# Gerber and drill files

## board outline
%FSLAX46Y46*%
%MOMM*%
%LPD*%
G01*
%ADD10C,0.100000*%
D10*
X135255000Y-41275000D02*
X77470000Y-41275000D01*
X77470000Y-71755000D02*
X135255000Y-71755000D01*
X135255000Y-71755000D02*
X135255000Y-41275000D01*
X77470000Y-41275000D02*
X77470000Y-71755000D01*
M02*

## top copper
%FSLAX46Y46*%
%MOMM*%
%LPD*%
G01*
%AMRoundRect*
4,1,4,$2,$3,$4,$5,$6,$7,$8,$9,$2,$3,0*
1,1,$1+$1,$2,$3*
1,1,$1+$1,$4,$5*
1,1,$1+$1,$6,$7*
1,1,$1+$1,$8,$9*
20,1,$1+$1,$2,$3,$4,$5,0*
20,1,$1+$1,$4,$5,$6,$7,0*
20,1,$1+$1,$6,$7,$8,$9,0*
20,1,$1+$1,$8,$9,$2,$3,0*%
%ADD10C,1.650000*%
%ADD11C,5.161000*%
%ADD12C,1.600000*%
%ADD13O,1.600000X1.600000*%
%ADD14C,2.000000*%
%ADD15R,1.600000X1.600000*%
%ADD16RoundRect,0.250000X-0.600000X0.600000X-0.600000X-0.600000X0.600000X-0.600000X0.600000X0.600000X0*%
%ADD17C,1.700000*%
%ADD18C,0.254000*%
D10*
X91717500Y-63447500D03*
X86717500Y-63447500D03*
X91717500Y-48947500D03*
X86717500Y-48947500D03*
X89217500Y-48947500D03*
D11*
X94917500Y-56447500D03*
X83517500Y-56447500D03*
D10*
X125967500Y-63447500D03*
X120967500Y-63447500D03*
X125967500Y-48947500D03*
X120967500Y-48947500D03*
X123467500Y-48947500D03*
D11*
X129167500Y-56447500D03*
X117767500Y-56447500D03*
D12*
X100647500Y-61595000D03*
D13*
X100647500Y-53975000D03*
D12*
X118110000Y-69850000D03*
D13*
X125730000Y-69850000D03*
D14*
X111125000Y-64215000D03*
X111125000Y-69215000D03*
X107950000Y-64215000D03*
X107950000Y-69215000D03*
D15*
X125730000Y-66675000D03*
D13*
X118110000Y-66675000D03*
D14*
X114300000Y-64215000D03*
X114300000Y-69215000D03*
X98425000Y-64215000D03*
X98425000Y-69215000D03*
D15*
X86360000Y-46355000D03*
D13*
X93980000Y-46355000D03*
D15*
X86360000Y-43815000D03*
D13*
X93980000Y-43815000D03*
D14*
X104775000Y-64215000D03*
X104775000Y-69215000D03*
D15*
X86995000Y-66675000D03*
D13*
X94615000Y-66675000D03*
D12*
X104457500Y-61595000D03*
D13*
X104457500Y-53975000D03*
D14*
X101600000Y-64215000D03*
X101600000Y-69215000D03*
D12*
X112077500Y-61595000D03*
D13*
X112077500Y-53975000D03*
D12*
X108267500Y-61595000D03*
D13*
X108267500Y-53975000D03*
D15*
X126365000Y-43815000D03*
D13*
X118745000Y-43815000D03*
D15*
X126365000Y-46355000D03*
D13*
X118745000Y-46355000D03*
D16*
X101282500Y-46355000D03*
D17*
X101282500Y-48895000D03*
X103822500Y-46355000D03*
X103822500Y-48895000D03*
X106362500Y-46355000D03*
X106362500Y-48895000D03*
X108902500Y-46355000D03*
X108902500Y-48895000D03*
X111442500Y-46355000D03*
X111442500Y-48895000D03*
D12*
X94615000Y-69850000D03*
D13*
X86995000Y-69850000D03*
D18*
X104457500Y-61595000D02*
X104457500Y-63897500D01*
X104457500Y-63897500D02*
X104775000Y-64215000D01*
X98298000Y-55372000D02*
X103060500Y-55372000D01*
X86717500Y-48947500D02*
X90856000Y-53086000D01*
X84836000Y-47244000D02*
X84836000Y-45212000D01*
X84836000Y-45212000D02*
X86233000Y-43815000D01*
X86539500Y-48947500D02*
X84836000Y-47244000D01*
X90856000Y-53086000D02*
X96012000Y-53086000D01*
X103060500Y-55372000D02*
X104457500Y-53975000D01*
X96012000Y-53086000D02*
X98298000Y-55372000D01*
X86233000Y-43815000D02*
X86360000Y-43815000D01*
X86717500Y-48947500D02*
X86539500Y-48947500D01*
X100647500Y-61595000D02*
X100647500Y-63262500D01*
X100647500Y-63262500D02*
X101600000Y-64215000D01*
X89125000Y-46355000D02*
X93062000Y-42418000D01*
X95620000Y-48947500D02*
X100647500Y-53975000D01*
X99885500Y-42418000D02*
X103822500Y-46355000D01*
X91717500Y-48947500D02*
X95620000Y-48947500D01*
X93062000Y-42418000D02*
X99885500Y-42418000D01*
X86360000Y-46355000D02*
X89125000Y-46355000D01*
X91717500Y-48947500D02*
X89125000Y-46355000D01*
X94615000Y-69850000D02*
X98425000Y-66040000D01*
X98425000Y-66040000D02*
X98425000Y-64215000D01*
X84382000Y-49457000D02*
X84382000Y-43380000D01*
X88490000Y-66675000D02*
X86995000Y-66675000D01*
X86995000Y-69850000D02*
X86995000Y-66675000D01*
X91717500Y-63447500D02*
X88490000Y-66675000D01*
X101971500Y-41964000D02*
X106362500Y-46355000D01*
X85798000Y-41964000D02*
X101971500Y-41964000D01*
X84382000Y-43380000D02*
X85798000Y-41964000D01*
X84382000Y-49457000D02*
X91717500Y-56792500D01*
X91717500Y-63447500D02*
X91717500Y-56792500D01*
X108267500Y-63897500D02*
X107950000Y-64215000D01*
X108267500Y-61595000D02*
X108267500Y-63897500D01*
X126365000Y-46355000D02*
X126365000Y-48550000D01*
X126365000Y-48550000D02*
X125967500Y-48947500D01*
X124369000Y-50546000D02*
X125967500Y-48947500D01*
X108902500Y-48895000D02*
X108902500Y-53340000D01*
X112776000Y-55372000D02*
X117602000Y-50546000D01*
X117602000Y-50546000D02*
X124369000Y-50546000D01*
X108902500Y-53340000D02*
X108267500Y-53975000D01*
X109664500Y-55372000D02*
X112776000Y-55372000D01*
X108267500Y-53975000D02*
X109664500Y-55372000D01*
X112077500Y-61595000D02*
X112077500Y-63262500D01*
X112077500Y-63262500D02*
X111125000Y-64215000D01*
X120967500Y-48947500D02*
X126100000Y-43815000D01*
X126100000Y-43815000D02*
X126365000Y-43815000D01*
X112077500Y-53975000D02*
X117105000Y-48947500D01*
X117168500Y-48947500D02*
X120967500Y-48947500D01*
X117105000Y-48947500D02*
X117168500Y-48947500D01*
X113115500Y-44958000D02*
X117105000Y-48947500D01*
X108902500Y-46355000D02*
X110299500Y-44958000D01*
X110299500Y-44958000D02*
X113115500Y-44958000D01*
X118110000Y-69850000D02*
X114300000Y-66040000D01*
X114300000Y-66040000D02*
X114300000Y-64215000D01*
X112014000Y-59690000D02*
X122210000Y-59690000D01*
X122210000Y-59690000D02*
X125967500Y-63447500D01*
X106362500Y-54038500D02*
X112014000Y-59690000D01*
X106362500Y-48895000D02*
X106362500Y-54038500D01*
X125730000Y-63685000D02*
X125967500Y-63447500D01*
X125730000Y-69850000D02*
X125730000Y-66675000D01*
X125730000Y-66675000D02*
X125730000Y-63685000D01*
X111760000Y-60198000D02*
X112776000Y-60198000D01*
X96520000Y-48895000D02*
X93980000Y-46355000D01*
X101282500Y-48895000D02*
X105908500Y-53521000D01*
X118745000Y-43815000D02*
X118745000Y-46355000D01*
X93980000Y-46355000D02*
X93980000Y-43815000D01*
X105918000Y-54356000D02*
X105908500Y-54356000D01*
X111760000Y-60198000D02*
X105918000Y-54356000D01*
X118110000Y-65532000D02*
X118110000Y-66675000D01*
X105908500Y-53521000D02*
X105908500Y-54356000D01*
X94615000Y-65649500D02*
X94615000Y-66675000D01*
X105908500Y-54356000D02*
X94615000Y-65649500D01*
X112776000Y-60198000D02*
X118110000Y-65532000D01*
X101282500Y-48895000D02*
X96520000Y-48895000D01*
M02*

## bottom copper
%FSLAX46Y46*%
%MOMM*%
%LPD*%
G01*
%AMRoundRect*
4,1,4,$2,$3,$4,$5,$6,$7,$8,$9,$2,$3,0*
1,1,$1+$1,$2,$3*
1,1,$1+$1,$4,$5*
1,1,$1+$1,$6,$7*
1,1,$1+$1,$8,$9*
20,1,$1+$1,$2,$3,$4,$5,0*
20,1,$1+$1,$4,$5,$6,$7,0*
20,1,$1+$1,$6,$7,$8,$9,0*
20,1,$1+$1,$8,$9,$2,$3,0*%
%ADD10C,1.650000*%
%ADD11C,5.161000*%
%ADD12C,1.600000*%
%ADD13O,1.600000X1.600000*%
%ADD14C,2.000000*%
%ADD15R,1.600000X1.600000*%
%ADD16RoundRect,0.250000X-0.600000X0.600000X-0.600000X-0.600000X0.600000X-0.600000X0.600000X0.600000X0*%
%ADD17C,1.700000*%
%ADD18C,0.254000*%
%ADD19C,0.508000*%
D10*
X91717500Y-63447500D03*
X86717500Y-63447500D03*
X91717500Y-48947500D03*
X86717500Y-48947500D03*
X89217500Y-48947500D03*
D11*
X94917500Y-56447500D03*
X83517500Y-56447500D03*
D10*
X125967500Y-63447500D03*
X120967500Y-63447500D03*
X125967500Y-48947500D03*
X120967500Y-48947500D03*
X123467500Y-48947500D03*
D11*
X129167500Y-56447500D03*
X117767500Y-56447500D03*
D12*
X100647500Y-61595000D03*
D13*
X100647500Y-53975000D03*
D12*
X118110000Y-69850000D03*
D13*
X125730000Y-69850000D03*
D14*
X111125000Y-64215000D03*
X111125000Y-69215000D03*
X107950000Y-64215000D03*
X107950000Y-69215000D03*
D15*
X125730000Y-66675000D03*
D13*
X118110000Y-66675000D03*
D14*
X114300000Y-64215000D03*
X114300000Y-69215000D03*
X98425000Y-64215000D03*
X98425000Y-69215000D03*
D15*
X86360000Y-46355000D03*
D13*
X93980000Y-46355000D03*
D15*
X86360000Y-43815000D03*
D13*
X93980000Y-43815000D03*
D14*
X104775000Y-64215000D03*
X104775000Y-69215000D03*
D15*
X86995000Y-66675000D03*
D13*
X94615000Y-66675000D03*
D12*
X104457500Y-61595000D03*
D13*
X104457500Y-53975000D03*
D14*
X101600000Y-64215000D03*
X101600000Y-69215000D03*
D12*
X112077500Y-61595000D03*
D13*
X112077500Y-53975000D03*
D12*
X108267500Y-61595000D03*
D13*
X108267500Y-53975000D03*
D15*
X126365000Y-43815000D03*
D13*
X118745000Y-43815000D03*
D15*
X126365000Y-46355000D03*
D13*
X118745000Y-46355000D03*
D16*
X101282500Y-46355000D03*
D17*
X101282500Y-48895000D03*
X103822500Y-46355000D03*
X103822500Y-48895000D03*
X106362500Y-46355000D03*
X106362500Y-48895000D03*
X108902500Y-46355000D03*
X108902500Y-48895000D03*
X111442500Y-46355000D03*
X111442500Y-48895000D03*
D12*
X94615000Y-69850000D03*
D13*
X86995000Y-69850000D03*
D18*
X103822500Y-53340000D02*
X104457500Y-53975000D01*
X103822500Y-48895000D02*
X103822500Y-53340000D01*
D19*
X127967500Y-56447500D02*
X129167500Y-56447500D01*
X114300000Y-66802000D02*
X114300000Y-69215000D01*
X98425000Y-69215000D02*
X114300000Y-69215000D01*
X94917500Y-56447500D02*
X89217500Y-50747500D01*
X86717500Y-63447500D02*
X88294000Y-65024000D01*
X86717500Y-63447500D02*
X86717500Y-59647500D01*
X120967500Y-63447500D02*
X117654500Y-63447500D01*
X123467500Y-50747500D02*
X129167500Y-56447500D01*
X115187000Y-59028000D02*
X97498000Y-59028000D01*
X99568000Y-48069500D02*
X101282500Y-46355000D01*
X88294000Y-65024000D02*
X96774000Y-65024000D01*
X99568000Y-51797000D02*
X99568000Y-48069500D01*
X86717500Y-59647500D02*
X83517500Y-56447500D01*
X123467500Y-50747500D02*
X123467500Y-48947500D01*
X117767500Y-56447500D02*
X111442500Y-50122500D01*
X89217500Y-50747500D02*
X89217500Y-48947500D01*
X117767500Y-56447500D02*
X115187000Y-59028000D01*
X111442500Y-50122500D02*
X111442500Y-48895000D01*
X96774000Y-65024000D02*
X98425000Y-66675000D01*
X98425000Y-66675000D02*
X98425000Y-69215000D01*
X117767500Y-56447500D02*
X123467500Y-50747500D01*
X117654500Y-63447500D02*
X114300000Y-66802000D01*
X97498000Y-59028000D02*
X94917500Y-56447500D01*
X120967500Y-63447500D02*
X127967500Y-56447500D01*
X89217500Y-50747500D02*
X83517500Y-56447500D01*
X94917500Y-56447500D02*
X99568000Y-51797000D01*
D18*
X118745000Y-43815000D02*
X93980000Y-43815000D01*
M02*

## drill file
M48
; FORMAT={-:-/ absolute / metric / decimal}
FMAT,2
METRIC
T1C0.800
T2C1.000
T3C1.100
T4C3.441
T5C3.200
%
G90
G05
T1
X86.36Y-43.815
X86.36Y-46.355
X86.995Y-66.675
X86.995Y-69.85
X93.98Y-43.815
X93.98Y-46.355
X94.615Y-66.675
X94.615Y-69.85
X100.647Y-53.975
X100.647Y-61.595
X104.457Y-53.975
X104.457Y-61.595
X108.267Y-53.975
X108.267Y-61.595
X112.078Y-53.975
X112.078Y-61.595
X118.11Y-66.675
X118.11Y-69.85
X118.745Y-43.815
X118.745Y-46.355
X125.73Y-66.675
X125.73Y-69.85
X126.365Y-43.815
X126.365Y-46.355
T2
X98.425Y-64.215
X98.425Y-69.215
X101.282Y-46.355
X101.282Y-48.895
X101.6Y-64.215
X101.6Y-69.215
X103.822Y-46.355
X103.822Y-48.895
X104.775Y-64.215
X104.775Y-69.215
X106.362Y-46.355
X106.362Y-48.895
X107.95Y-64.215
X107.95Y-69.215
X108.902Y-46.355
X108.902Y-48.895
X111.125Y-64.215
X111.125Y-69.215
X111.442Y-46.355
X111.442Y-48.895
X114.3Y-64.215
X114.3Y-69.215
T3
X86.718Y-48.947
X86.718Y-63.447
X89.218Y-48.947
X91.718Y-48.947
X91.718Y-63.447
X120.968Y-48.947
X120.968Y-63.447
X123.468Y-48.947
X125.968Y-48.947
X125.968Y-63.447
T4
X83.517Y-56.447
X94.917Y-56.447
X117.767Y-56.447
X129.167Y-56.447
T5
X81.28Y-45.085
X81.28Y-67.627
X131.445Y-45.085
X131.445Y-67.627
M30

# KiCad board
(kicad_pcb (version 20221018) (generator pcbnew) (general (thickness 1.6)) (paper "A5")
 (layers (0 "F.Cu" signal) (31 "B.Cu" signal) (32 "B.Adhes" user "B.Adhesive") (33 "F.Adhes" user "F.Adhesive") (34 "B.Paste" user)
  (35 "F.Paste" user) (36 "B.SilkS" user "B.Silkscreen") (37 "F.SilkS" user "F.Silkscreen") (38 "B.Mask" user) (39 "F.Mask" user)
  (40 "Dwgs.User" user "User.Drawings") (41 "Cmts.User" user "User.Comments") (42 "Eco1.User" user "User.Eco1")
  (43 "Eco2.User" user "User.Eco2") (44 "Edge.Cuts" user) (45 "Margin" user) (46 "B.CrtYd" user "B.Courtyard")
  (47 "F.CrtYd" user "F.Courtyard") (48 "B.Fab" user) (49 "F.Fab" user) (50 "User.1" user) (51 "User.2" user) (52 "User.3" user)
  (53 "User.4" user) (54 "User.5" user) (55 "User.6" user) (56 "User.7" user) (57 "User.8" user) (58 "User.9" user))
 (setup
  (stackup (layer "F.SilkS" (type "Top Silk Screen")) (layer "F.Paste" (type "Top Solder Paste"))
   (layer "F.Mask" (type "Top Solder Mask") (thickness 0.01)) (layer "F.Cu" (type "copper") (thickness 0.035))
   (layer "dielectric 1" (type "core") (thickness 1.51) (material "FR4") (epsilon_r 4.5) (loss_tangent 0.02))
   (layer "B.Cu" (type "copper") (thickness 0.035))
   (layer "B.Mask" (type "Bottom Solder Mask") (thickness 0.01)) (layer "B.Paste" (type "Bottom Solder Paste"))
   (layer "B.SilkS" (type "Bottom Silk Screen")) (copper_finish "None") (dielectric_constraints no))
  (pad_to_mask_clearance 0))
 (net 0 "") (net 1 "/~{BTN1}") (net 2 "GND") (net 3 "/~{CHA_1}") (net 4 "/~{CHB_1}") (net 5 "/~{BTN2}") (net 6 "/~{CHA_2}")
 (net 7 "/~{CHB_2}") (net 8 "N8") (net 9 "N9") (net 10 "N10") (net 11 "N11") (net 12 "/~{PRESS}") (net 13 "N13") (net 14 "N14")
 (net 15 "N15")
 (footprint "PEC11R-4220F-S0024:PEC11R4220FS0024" (layer "F.Cu") (at 91.7175 63.4475 180)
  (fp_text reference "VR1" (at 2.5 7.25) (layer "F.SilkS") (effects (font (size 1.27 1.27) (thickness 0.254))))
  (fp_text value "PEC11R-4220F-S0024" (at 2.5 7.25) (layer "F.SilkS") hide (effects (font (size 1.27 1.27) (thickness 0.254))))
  (pad "1" thru_hole circle (at 0 0 270) (size 1.65 1.65) (drill 1.1) (layers "*.Cu" "*.Mask" "F.SilkS") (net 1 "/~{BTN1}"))
  (pad "2" thru_hole circle (at 5 0 270) (size 1.65 1.65) (drill 1.1) (layers "*.Cu" "*.Mask" "F.SilkS") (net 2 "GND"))
  (pad "A1" thru_hole circle (at 0 14.5 270) (size 1.65 1.65) (drill 1.1) (layers "*.Cu" "*.Mask" "F.SilkS") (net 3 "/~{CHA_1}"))
  (pad "B1" thru_hole circle (at 5 14.5 270) (size 1.65 1.65) (drill 1.1) (layers "*.Cu" "*.Mask" "F.SilkS") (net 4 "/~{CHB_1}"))
  (pad "C1" thru_hole circle (at 2.5 14.5 270) (size 1.65 1.65) (drill 1.1) (layers "*.Cu" "*.Mask" "F.SilkS") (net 2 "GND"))
  (pad "MH1" thru_hole circle (at -3.2 7 270) (size 5.161 5.161) (drill 3.4409) (layers "*.Cu" "*.Mask" "F.SilkS") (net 2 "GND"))
  (pad "MH2" thru_hole circle (at 8.2 7 270) (size 5.161 5.161) (drill 3.4409) (layers "*.Cu" "*.Mask" "F.SilkS") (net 2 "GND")))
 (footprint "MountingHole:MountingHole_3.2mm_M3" (layer "F.Cu") (at 131.445 67.6275)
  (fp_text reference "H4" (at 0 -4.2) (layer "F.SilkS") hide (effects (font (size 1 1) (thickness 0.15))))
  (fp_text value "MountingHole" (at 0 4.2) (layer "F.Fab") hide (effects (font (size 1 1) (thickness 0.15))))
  (pad "" np_thru_hole circle (at 0 0) (size 3.2 3.2) (drill 3.2) (layers "*.Cu" "*.Mask")))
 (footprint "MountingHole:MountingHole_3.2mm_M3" (layer "F.Cu") (at 81.28 45.085)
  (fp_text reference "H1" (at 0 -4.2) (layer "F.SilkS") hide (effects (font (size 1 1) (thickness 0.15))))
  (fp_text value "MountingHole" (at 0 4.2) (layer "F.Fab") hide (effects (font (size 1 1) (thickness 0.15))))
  (pad "" np_thru_hole circle (at 0 0) (size 3.2 3.2) (drill 3.2) (layers "*.Cu" "*.Mask")))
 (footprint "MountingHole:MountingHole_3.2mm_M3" (layer "F.Cu") (at 131.445 45.085)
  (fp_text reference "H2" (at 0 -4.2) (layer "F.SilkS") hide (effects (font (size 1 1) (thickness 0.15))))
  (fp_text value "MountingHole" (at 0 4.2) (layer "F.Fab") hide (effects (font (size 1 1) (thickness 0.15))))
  (pad "" np_thru_hole circle (at 0 0) (size 3.2 3.2) (drill 3.2) (layers "*.Cu" "*.Mask")))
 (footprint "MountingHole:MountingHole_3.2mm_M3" (layer "F.Cu") (at 81.28 67.6275)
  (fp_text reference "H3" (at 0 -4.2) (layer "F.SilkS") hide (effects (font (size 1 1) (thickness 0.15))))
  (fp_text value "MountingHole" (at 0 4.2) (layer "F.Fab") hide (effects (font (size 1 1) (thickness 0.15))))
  (pad "" np_thru_hole circle (at 0 0) (size 3.2 3.2) (drill 3.2) (layers "*.Cu" "*.Mask")))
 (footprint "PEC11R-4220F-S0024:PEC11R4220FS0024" (layer "F.Cu") (at 125.9675 63.4475 180)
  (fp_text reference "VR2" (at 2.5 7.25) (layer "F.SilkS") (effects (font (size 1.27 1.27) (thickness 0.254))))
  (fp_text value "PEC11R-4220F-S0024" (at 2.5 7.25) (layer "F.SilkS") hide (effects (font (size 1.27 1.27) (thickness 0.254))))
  (pad "1" thru_hole circle (at 0 0 270) (size 1.65 1.65) (drill 1.1) (layers "*.Cu" "*.Mask" "F.SilkS") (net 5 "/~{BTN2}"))
  (pad "2" thru_hole circle (at 5 0 270) (size 1.65 1.65) (drill 1.1) (layers "*.Cu" "*.Mask" "F.SilkS") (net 2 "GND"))
  (pad "A1" thru_hole circle (at 0 14.5 270) (size 1.65 1.65) (drill 1.1) (layers "*.Cu" "*.Mask" "F.SilkS") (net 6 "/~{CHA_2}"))
  (pad "B1" thru_hole circle (at 5 14.5 270) (size 1.65 1.65) (drill 1.1) (layers "*.Cu" "*.Mask" "F.SilkS") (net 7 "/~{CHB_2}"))
  (pad "C1" thru_hole circle (at 2.5 14.5 270) (size 1.65 1.65) (drill 1.1) (layers "*.Cu" "*.Mask" "F.SilkS") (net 2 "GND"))
  (pad "MH1" thru_hole circle (at -3.2 7 270) (size 5.161 5.161) (drill 3.4409) (layers "*.Cu" "*.Mask" "F.SilkS") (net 2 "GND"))
  (pad "MH2" thru_hole circle (at 8.2 7 270) (size 5.161 5.161) (drill 3.4409) (layers "*.Cu" "*.Mask" "F.SilkS") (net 2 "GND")))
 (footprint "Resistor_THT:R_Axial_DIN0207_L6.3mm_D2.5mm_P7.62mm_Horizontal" (layer "B.Cu") (at 100.6475 61.595 90)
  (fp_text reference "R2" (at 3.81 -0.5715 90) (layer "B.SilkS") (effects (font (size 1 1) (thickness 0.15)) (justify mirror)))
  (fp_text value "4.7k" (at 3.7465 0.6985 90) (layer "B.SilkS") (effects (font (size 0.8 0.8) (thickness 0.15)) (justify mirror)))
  (pad "1" thru_hole circle (at 0 0 90) (size 1.6 1.6) (drill 0.8) (layers "*.Cu" "*.Mask") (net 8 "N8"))
  (pad "2" thru_hole oval (at 7.62 0 90) (size 1.6 1.6) (drill 0.8) (layers "*.Cu" "*.Mask") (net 3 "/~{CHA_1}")))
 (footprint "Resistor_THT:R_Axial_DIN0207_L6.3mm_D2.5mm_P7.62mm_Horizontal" (layer "B.Cu") (at 118.11 69.85)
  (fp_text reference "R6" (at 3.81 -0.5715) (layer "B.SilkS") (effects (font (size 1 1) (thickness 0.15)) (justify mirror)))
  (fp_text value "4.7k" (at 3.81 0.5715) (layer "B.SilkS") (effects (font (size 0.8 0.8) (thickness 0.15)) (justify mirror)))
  (pad "1" thru_hole circle (at 0 0) (size 1.6 1.6) (drill 0.8) (layers "*.Cu" "*.Mask") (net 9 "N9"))
  (pad "2" thru_hole oval (at 7.62 0) (size 1.6 1.6) (drill 0.8) (layers "*.Cu" "*.Mask") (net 5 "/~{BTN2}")))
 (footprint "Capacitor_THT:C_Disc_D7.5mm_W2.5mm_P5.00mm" (layer "B.Cu") (at 111.125 64.215 -90)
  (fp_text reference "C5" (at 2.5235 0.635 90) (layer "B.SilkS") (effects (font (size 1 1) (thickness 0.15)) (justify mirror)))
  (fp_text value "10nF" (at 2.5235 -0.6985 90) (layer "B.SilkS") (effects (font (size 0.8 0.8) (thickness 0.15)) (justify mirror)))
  (pad "1" thru_hole circle (at 0 0 270) (size 2 2) (drill 1) (layers "*.Cu" "*.Mask") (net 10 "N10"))
  (pad "2" thru_hole circle (at 5 0 270) (size 2 2) (drill 1) (layers "*.Cu" "*.Mask") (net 2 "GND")))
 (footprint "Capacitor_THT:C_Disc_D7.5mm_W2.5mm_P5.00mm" (layer "B.Cu") (at 107.95 64.215 -90)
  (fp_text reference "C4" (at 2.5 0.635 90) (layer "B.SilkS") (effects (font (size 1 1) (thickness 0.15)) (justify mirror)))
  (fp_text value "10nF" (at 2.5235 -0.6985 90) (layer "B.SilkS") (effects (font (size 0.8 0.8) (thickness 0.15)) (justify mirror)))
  (pad "1" thru_hole circle (at 0 0 270) (size 2 2) (drill 1) (layers "*.Cu" "*.Mask") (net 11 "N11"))
  (pad "2" thru_hole circle (at 5 0 270) (size 2 2) (drill 1) (layers "*.Cu" "*.Mask") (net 2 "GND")))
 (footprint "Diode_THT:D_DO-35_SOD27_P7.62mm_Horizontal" (layer "B.Cu") (at 125.73 66.675 180)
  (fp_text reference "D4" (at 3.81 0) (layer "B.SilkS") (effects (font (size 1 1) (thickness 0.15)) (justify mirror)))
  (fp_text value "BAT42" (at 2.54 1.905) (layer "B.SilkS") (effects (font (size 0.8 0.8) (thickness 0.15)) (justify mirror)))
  (pad "1" thru_hole rect (at 0 0 180) (size 1.6 1.6) (drill 0.8) (layers "*.Cu" "*.Mask") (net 5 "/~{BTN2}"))
  (pad "2" thru_hole oval (at 7.62 0 180) (size 1.6 1.6) (drill 0.8) (layers "*.Cu" "*.Mask") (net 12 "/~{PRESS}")))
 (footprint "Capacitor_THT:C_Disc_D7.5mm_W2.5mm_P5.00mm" (layer "B.Cu") (at 114.3 64.215 -90)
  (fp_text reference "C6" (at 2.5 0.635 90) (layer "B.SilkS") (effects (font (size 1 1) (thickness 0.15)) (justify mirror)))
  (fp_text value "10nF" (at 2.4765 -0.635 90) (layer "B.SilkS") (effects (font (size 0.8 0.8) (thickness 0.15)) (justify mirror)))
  (pad "1" thru_hole circle (at 0 0 270) (size 2 2) (drill 1) (layers "*.Cu" "*.Mask") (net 9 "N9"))
  (pad "2" thru_hole circle (at 5 0 270) (size 2 2) (drill 1) (layers "*.Cu" "*.Mask") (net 2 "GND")))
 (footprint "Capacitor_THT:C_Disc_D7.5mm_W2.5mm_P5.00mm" (layer "B.Cu") (at 98.425 64.215 -90)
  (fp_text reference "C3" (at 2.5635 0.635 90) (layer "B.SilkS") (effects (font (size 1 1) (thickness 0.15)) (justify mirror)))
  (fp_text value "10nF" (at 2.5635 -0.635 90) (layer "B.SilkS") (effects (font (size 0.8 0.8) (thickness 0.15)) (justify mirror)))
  (pad "1" thru_hole circle (at 0 0 270) (size 2 2) (drill 1) (layers "*.Cu" "*.Mask") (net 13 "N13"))
  (pad "2" thru_hole circle (at 5 0 270) (size 2 2) (drill 1) (layers "*.Cu" "*.Mask") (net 2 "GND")))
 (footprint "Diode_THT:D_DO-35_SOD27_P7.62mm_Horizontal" (layer "B.Cu") (at 86.36 46.355)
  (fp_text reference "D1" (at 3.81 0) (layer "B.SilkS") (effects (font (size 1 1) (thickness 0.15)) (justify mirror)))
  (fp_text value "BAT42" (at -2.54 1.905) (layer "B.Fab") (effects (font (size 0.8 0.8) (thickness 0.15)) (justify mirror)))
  (pad "1" thru_hole rect (at 0 0) (size 1.6 1.6) (drill 0.8) (layers "*.Cu" "*.Mask") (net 3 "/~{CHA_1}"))
  (pad "2" thru_hole oval (at 7.62 0) (size 1.6 1.6) (drill 0.8) (layers "*.Cu" "*.Mask") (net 12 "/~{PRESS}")))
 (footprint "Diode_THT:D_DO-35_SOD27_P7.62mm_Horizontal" (layer "B.Cu") (at 86.36 43.815)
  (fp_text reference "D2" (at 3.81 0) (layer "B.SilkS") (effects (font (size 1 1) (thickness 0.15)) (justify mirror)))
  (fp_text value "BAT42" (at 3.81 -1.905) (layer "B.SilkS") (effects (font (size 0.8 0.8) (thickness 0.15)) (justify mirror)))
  (pad "1" thru_hole rect (at 0 0) (size 1.6 1.6) (drill 0.8) (layers "*.Cu" "*.Mask") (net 4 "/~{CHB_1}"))
  (pad "2" thru_hole oval (at 7.62 0) (size 1.6 1.6) (drill 0.8) (layers "*.Cu" "*.Mask") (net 12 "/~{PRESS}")))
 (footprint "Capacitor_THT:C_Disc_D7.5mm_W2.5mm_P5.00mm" (layer "B.Cu") (at 104.775 64.215 -90)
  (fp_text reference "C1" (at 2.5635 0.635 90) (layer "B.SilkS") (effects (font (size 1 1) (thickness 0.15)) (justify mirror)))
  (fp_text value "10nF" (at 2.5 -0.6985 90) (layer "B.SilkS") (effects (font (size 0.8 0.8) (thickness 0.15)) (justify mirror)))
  (pad "1" thru_hole circle (at 0 0 270) (size 2 2) (drill 1) (layers "*.Cu" "*.Mask") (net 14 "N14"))
  (pad "2" thru_hole circle (at 5 0 270) (size 2 2) (drill 1) (layers "*.Cu" "*.Mask") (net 2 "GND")))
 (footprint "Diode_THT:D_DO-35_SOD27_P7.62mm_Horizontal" (layer "B.Cu") (at 86.995 66.675)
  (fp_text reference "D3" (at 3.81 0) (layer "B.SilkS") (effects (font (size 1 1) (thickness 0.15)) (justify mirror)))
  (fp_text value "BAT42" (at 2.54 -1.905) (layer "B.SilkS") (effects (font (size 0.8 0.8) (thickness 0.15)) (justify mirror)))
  (pad "1" thru_hole rect (at 0 0) (size 1.6 1.6) (drill 0.8) (layers "*.Cu" "*.Mask") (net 1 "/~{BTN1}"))
  (pad "2" thru_hole oval (at 7.62 0) (size 1.6 1.6) (drill 0.8) (layers "*.Cu" "*.Mask") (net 12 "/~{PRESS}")))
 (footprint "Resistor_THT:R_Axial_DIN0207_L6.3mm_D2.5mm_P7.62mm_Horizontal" (layer "B.Cu") (at 104.4575 61.595 90)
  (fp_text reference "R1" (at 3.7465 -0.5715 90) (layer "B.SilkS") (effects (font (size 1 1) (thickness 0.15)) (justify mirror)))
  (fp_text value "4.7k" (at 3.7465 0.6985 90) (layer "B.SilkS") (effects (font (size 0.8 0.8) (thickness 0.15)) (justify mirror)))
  (pad "1" thru_hole circle (at 0 0 90) (size 1.6 1.6) (drill 0.8) (layers "*.Cu" "*.Mask") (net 14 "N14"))
  (pad "2" thru_hole oval (at 7.62 0 90) (size 1.6 1.6) (drill 0.8) (layers "*.Cu" "*.Mask") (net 4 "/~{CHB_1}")))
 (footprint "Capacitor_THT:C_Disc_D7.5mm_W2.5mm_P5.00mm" (layer "B.Cu") (at 101.6 64.215 -90)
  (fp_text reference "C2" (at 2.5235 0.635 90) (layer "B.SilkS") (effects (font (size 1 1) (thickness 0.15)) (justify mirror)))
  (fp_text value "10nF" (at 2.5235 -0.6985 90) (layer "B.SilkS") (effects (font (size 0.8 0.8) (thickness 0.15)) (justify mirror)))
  (pad "1" thru_hole circle (at 0 0 270) (size 2 2) (drill 1) (layers "*.Cu" "*.Mask") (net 8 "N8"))
  (pad "2" thru_hole circle (at 5 0 270) (size 2 2) (drill 1) (layers "*.Cu" "*.Mask") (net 2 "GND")))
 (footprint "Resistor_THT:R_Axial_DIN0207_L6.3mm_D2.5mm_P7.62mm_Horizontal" (layer "B.Cu") (at 112.0775 61.595 90)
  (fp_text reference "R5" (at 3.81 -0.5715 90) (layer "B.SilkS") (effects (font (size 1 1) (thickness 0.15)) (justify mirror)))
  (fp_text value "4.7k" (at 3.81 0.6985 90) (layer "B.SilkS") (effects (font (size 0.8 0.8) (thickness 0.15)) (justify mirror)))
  (pad "1" thru_hole circle (at 0 0 90) (size 1.6 1.6) (drill 0.8) (layers "*.Cu" "*.Mask") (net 10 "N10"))
  (pad "2" thru_hole oval (at 7.62 0 90) (size 1.6 1.6) (drill 0.8) (layers "*.Cu" "*.Mask") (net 7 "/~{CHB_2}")))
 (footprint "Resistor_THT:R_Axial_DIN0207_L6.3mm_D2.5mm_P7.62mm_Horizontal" (layer "B.Cu") (at 108.2675 61.595 90)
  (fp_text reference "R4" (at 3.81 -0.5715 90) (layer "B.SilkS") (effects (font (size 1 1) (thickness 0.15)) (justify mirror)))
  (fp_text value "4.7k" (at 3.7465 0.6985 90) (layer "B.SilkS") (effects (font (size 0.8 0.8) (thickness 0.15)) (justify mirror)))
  (pad "1" thru_hole circle (at 0 0 90) (size 1.6 1.6) (drill 0.8) (layers "*.Cu" "*.Mask") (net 11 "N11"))
  (pad "2" thru_hole oval (at 7.62 0 90) (size 1.6 1.6) (drill 0.8) (layers "*.Cu" "*.Mask") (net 6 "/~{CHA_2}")))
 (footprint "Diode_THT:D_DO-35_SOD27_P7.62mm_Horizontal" (layer "B.Cu") (at 126.365 43.815 180)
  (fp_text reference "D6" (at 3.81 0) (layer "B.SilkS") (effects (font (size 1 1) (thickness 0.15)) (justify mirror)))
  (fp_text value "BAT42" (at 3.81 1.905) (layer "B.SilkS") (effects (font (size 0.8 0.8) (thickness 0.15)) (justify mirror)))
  (pad "1" thru_hole rect (at 0 0 180) (size 1.6 1.6) (drill 0.8) (layers "*.Cu" "*.Mask") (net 7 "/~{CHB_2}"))
  (pad "2" thru_hole oval (at 7.62 0 180) (size 1.6 1.6) (drill 0.8) (layers "*.Cu" "*.Mask") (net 12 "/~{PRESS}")))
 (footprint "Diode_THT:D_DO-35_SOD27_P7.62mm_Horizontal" (layer "B.Cu") (at 126.365 46.355 180)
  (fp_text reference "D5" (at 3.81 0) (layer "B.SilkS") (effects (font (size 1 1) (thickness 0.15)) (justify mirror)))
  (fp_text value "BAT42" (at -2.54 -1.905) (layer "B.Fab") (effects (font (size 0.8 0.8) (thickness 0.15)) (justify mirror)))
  (pad "1" thru_hole rect (at 0 0 180) (size 1.6 1.6) (drill 0.8) (layers "*.Cu" "*.Mask") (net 6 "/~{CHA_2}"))
  (pad "2" thru_hole oval (at 7.62 0 180) (size 1.6 1.6) (drill 0.8) (layers "*.Cu" "*.Mask") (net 12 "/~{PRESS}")))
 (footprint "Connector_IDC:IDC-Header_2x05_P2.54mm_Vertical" (layer "B.Cu") (at 101.2825 46.355 -90)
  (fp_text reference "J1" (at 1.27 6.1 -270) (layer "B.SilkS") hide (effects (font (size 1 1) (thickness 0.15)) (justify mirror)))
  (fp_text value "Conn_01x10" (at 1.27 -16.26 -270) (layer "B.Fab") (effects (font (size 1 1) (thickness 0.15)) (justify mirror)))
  (pad "1" thru_hole roundrect (at 0 0 270) (size 1.7 1.7) (drill 1) (layers "*.Cu" "*.Mask") (roundrect_rratio 0.1470588235) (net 2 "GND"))
  (pad "2" thru_hole circle (at 2.54 0 270) (size 1.7 1.7) (drill 1) (layers "*.Cu" "*.Mask") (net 12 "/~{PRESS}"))
  (pad "3" thru_hole circle (at 0 -2.54 270) (size 1.7 1.7) (drill 1) (layers "*.Cu" "*.Mask") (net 3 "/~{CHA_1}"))
  (pad "4" thru_hole circle (at 2.54 -2.54 270) (size 1.7 1.7) (drill 1) (layers "*.Cu" "*.Mask") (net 4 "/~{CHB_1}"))
  (pad "5" thru_hole circle (at 0 -5.08 270) (size 1.7 1.7) (drill 1) (layers "*.Cu" "*.Mask") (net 1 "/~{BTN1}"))
  (pad "6" thru_hole circle (at 2.54 -5.08 270) (size 1.7 1.7) (drill 1) (layers "*.Cu" "*.Mask") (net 5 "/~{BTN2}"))
  (pad "7" thru_hole circle (at 0 -7.62 270) (size 1.7 1.7) (drill 1) (layers "*.Cu" "*.Mask") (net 7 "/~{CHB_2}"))
  (pad "8" thru_hole circle (at 2.54 -7.62 270) (size 1.7 1.7) (drill 1) (layers "*.Cu" "*.Mask") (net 6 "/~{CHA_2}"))
  (pad "9" thru_hole circle (at 0 -10.16 270) (size 1.7 1.7) (drill 1) (layers "*.Cu" "*.Mask") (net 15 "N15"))
  (pad "10" thru_hole circle (at 2.54 -10.16 270) (size 1.7 1.7) (drill 1) (layers "*.Cu" "*.Mask") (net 2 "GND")))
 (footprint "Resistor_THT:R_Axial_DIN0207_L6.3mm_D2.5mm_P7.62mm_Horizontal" (layer "B.Cu") (at 94.615 69.85 180)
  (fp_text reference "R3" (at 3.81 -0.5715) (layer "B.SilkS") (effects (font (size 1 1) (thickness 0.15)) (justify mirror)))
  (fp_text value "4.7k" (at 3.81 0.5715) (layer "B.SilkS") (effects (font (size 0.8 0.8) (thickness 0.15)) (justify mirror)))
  (pad "1" thru_hole circle (at 0 0 180) (size 1.6 1.6) (drill 0.8) (layers "*.Cu" "*.Mask") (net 13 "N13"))
  (pad "2" thru_hole oval (at 7.62 0 180) (size 1.6 1.6) (drill 0.8) (layers "*.Cu" "*.Mask") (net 1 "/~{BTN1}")))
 (gr_line (start 135.255 41.275) (end 77.47 41.275) (stroke (width 0.1) (type default)) (layer "Edge.Cuts"))
 (gr_line (start 77.47 71.755) (end 135.255 71.755) (stroke (width 0.1) (type default)) (layer "Edge.Cuts"))
 (gr_line (start 135.255 71.755) (end 135.255 41.275) (stroke (width 0.1) (type default)) (layer "Edge.Cuts"))
 (gr_line (start 77.47 41.275) (end 77.47 71.755) (stroke (width 0.1) (type default)) (layer "Edge.Cuts"))
 (segment (start 104.4575 61.595) (end 104.4575 63.8975) (width 0.254) (layer "F.Cu") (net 14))
 (segment (start 104.4575 63.8975) (end 104.775 64.215) (width 0.254) (layer "F.Cu") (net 14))
 (segment (start 98.298 55.372) (end 103.0605 55.372) (width 0.254) (layer "F.Cu") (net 4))
 (segment (start 86.7175 48.9475) (end 90.856 53.086) (width 0.254) (layer "F.Cu") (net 4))
 (segment (start 84.836 47.244) (end 84.836 45.212) (width 0.254) (layer "F.Cu") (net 4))
 (segment (start 84.836 45.212) (end 86.233 43.815) (width 0.254) (layer "F.Cu") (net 4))
 (segment (start 86.5395 48.9475) (end 84.836 47.244) (width 0.254) (layer "F.Cu") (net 4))
 (segment (start 90.856 53.086) (end 96.012 53.086) (width 0.254) (layer "F.Cu") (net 4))
 (segment (start 103.0605 55.372) (end 104.4575 53.975) (width 0.254) (layer "F.Cu") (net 4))
 (segment (start 96.012 53.086) (end 98.298 55.372) (width 0.254) (layer "F.Cu") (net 4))
 (segment (start 86.233 43.815) (end 86.36 43.815) (width 0.254) (layer "F.Cu") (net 4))
 (segment (start 86.7175 48.9475) (end 86.5395 48.9475) (width 0.254) (layer "F.Cu") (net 4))
 (segment (start 103.8225 53.34) (end 104.4575 53.975) (width 0.254) (layer "B.Cu") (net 4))
 (segment (start 103.8225 48.895) (end 103.8225 53.34) (width 0.254) (layer "B.Cu") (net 4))
 (segment (start 100.6475 61.595) (end 100.6475 63.2625) (width 0.254) (layer "F.Cu") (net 8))
 (segment (start 100.6475 63.2625) (end 101.6 64.215) (width 0.254) (layer "F.Cu") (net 8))
 (segment (start 89.125 46.355) (end 93.062 42.418) (width 0.254) (layer "F.Cu") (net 3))
 (segment (start 95.62 48.9475) (end 100.6475 53.975) (width 0.254) (layer "F.Cu") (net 3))
 (segment (start 99.8855 42.418) (end 103.8225 46.355) (width 0.254) (layer "F.Cu") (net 3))
 (segment (start 91.7175 48.9475) (end 95.62 48.9475) (width 0.254) (layer "F.Cu") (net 3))
 (segment (start 93.062 42.418) (end 99.8855 42.418) (width 0.254) (layer "F.Cu") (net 3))
 (segment (start 86.36 46.355) (end 89.125 46.355) (width 0.254) (layer "F.Cu") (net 3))
 (segment (start 91.7175 48.9475) (end 89.125 46.355) (width 0.254) (layer "F.Cu") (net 3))
 (segment (start 94.615 69.85) (end 98.425 66.04) (width 0.254) (layer "F.Cu") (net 13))
 (segment (start 98.425 66.04) (end 98.425 64.215) (width 0.254) (layer "F.Cu") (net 13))
 (segment (start 84.382 49.457) (end 84.382 43.38) (width 0.254) (layer "F.Cu") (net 1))
 (segment (start 88.49 66.675) (end 86.995 66.675) (width 0.254) (layer "F.Cu") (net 1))
 (segment (start 86.995 69.85) (end 86.995 66.675) (width 0.254) (layer "F.Cu") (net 1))
 (segment (start 91.7175 63.4475) (end 88.49 66.675) (width 0.254) (layer "F.Cu") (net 1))
 (segment (start 101.9715 41.964) (end 106.3625 46.355) (width 0.254) (layer "F.Cu") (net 1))
 (segment (start 85.798 41.964) (end 101.9715 41.964) (width 0.254) (layer "F.Cu") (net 1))
 (segment (start 84.382 43.38) (end 85.798 41.964) (width 0.254) (layer "F.Cu") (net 1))
 (segment (start 84.382 49.457) (end 91.7175 56.7925) (width 0.254) (layer "F.Cu") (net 1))
 (segment (start 91.7175 63.4475) (end 91.7175 56.7925) (width 0.254) (layer "F.Cu") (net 1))
 (segment (start 108.2675 63.8975) (end 107.95 64.215) (width 0.254) (layer "F.Cu") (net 11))
 (segment (start 108.2675 61.595) (end 108.2675 63.8975) (width 0.254) (layer "F.Cu") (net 11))
 (segment (start 126.365 46.355) (end 126.365 48.55) (width 0.254) (layer "F.Cu") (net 6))
 (segment (start 126.365 48.55) (end 125.9675 48.9475) (width 0.254) (layer "F.Cu") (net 6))
 (segment (start 124.369 50.546) (end 125.9675 48.9475) (width 0.254) (layer "F.Cu") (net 6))
 (segment (start 108.9025 48.895) (end 108.9025 53.34) (width 0.254) (layer "F.Cu") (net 6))
 (segment (start 112.776 55.372) (end 117.602 50.546) (width 0.254) (layer "F.Cu") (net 6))
 (segment (start 117.602 50.546) (end 124.369 50.546) (width 0.254) (layer "F.Cu") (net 6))
 (segment (start 108.9025 53.34) (end 108.2675 53.975) (width 0.254) (layer "F.Cu") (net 6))
 (segment (start 109.6645 55.372) (end 112.776 55.372) (width 0.254) (layer "F.Cu") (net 6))
 (segment (start 108.2675 53.975) (end 109.6645 55.372) (width 0.254) (layer "F.Cu") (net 6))
 (segment (start 112.0775 61.595) (end 112.0775 63.2625) (width 0.254) (layer "F.Cu") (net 10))
 (segment (start 112.0775 63.2625) (end 111.125 64.215) (width 0.254) (layer "F.Cu") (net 10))
 (segment (start 120.9675 48.9475) (end 126.1 43.815) (width 0.254) (layer "F.Cu") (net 7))
 (segment (start 126.1 43.815) (end 126.365 43.815) (width 0.254) (layer "F.Cu") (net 7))
 (segment (start 112.0775 53.975) (end 117.105 48.9475) (width 0.254) (layer "F.Cu") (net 7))
 (segment (start 117.1685 48.9475) (end 120.9675 48.9475) (width 0.254) (layer "F.Cu") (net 7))
 (segment (start 117.105 48.9475) (end 117.1685 48.9475) (width 0.254) (layer "F.Cu") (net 7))
 (segment (start 113.1155 44.958) (end 117.105 48.9475) (width 0.254) (layer "F.Cu") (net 7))
 (segment (start 108.9025 46.355) (end 110.2995 44.958) (width 0.254) (layer "F.Cu") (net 7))
 (segment (start 110.2995 44.958) (end 113.1155 44.958) (width 0.254) (layer "F.Cu") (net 7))
 (segment (start 118.11 69.85) (end 114.3 66.04) (width 0.254) (layer "F.Cu") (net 9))
 (segment (start 114.3 66.04) (end 114.3 64.215) (width 0.254) (layer "F.Cu") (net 9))
 (segment (start 112.014 59.69) (end 122.21 59.69) (width 0.254) (layer "F.Cu") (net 5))
 (segment (start 122.21 59.69) (end 125.9675 63.4475) (width 0.254) (layer "F.Cu") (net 5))
 (segment (start 106.3625 54.0385) (end 112.014 59.69) (width 0.254) (layer "F.Cu") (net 5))
 (segment (start 106.3625 48.895) (end 106.3625 54.0385) (width 0.254) (layer "F.Cu") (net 5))
 (segment (start 125.73 63.685) (end 125.9675 63.4475) (width 0.254) (layer "F.Cu") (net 5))
 (segment (start 125.73 69.85) (end 125.73 66.675) (width 0.254) (layer "F.Cu") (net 5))
 (segment (start 125.73 66.675) (end 125.73 63.685) (width 0.254) (layer "F.Cu") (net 5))
 (segment (start 127.9675 56.4475) (end 129.1675 56.4475) (width 0.508) (layer "B.Cu") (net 2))
 (segment (start 114.3 66.802) (end 114.3 69.215) (width 0.508) (layer "B.Cu") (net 2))
 (segment (start 98.425 69.215) (end 114.3 69.215) (width 0.508) (layer "B.Cu") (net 2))
 (segment (start 94.9175 56.4475) (end 89.2175 50.7475) (width 0.508) (layer "B.Cu") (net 2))
 (segment (start 86.7175 63.4475) (end 88.294 65.024) (width 0.508) (layer "B.Cu") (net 2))
 (segment (start 86.7175 63.4475) (end 86.7175 59.6475) (width 0.508) (layer "B.Cu") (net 2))
 (segment (start 120.9675 63.4475) (end 117.6545 63.4475) (width 0.508) (layer "B.Cu") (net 2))
 (segment (start 123.4675 50.7475) (end 129.1675 56.4475) (width 0.508) (layer "B.Cu") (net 2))
 (segment (start 115.187 59.028) (end 97.498 59.028) (width 0.508) (layer "B.Cu") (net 2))
 (segment (start 99.568 48.0695) (end 101.2825 46.355) (width 0.508) (layer "B.Cu") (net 2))
 (segment (start 88.294 65.024) (end 96.774 65.024) (width 0.508) (layer "B.Cu") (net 2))
 (segment (start 99.568 51.797) (end 99.568 48.0695) (width 0.508) (layer "B.Cu") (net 2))
 (segment (start 86.7175 59.6475) (end 83.5175 56.4475) (width 0.508) (layer "B.Cu") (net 2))
 (segment (start 123.4675 50.7475) (end 123.4675 48.9475) (width 0.508) (layer "B.Cu") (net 2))
 (segment (start 117.7675 56.4475) (end 111.4425 50.1225) (width 0.508) (layer "B.Cu") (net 2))
 (segment (start 89.2175 50.7475) (end 89.2175 48.9475) (width 0.508) (layer "B.Cu") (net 2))
 (segment (start 117.7675 56.4475) (end 115.187 59.028) (width 0.508) (layer "B.Cu") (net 2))
 (segment (start 111.4425 50.1225) (end 111.4425 48.895) (width 0.508) (layer "B.Cu") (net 2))
 (segment (start 96.774 65.024) (end 98.425 66.675) (width 0.508) (layer "B.Cu") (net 2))
 (segment (start 98.425 66.675) (end 98.425 69.215) (width 0.508) (layer "B.Cu") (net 2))
 (segment (start 117.7675 56.4475) (end 123.4675 50.7475) (width 0.508) (layer "B.Cu") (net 2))
 (segment (start 117.6545 63.4475) (end 114.3 66.802) (width 0.508) (layer "B.Cu") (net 2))
 (segment (start 97.498 59.028) (end 94.9175 56.4475) (width 0.508) (layer "B.Cu") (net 2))
 (segment (start 120.9675 63.4475) (end 127.9675 56.4475) (width 0.508) (layer "B.Cu") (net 2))
 (segment (start 89.2175 50.7475) (end 83.5175 56.4475) (width 0.508) (layer "B.Cu") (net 2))
 (segment (start 94.9175 56.4475) (end 99.568 51.797) (width 0.508) (layer "B.Cu") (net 2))
 (segment (start 111.76 60.198) (end 112.776 60.198) (width 0.254) (layer "F.Cu") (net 12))
 (segment (start 96.52 48.895) (end 93.98 46.355) (width 0.254) (layer "F.Cu") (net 12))
 (segment (start 101.2825 48.895) (end 105.9085 53.521) (width 0.254) (layer "F.Cu") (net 12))
 (segment (start 118.745 43.815) (end 118.745 46.355) (width 0.254) (layer "F.Cu") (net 12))
 (segment (start 93.98 46.355) (end 93.98 43.815) (width 0.254) (layer "F.Cu") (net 12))
 (segment (start 105.918 54.356) (end 105.9085 54.356) (width 0.254) (layer "F.Cu") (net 12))
 (segment (start 111.76 60.198) (end 105.918 54.356) (width 0.254) (layer "F.Cu") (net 12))
 (segment (start 118.11 65.532) (end 118.11 66.675) (width 0.254) (layer "F.Cu") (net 12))
 (segment (start 105.9085 53.521) (end 105.9085 54.356) (width 0.254) (layer "F.Cu") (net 12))
 (segment (start 94.615 65.6495) (end 94.615 66.675) (width 0.254) (layer "F.Cu") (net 12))
 (segment (start 105.9085 54.356) (end 94.615 65.6495) (width 0.254) (layer "F.Cu") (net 12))
 (segment (start 112.776 60.198) (end 118.11 65.532) (width 0.254) (layer "F.Cu") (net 12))
 (segment (start 101.2825 48.895) (end 96.52 48.895) (width 0.254) (layer "F.Cu") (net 12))
 (segment (start 118.745 43.815) (end 93.98 43.815) (width 0.254) (layer "B.Cu") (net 12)))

